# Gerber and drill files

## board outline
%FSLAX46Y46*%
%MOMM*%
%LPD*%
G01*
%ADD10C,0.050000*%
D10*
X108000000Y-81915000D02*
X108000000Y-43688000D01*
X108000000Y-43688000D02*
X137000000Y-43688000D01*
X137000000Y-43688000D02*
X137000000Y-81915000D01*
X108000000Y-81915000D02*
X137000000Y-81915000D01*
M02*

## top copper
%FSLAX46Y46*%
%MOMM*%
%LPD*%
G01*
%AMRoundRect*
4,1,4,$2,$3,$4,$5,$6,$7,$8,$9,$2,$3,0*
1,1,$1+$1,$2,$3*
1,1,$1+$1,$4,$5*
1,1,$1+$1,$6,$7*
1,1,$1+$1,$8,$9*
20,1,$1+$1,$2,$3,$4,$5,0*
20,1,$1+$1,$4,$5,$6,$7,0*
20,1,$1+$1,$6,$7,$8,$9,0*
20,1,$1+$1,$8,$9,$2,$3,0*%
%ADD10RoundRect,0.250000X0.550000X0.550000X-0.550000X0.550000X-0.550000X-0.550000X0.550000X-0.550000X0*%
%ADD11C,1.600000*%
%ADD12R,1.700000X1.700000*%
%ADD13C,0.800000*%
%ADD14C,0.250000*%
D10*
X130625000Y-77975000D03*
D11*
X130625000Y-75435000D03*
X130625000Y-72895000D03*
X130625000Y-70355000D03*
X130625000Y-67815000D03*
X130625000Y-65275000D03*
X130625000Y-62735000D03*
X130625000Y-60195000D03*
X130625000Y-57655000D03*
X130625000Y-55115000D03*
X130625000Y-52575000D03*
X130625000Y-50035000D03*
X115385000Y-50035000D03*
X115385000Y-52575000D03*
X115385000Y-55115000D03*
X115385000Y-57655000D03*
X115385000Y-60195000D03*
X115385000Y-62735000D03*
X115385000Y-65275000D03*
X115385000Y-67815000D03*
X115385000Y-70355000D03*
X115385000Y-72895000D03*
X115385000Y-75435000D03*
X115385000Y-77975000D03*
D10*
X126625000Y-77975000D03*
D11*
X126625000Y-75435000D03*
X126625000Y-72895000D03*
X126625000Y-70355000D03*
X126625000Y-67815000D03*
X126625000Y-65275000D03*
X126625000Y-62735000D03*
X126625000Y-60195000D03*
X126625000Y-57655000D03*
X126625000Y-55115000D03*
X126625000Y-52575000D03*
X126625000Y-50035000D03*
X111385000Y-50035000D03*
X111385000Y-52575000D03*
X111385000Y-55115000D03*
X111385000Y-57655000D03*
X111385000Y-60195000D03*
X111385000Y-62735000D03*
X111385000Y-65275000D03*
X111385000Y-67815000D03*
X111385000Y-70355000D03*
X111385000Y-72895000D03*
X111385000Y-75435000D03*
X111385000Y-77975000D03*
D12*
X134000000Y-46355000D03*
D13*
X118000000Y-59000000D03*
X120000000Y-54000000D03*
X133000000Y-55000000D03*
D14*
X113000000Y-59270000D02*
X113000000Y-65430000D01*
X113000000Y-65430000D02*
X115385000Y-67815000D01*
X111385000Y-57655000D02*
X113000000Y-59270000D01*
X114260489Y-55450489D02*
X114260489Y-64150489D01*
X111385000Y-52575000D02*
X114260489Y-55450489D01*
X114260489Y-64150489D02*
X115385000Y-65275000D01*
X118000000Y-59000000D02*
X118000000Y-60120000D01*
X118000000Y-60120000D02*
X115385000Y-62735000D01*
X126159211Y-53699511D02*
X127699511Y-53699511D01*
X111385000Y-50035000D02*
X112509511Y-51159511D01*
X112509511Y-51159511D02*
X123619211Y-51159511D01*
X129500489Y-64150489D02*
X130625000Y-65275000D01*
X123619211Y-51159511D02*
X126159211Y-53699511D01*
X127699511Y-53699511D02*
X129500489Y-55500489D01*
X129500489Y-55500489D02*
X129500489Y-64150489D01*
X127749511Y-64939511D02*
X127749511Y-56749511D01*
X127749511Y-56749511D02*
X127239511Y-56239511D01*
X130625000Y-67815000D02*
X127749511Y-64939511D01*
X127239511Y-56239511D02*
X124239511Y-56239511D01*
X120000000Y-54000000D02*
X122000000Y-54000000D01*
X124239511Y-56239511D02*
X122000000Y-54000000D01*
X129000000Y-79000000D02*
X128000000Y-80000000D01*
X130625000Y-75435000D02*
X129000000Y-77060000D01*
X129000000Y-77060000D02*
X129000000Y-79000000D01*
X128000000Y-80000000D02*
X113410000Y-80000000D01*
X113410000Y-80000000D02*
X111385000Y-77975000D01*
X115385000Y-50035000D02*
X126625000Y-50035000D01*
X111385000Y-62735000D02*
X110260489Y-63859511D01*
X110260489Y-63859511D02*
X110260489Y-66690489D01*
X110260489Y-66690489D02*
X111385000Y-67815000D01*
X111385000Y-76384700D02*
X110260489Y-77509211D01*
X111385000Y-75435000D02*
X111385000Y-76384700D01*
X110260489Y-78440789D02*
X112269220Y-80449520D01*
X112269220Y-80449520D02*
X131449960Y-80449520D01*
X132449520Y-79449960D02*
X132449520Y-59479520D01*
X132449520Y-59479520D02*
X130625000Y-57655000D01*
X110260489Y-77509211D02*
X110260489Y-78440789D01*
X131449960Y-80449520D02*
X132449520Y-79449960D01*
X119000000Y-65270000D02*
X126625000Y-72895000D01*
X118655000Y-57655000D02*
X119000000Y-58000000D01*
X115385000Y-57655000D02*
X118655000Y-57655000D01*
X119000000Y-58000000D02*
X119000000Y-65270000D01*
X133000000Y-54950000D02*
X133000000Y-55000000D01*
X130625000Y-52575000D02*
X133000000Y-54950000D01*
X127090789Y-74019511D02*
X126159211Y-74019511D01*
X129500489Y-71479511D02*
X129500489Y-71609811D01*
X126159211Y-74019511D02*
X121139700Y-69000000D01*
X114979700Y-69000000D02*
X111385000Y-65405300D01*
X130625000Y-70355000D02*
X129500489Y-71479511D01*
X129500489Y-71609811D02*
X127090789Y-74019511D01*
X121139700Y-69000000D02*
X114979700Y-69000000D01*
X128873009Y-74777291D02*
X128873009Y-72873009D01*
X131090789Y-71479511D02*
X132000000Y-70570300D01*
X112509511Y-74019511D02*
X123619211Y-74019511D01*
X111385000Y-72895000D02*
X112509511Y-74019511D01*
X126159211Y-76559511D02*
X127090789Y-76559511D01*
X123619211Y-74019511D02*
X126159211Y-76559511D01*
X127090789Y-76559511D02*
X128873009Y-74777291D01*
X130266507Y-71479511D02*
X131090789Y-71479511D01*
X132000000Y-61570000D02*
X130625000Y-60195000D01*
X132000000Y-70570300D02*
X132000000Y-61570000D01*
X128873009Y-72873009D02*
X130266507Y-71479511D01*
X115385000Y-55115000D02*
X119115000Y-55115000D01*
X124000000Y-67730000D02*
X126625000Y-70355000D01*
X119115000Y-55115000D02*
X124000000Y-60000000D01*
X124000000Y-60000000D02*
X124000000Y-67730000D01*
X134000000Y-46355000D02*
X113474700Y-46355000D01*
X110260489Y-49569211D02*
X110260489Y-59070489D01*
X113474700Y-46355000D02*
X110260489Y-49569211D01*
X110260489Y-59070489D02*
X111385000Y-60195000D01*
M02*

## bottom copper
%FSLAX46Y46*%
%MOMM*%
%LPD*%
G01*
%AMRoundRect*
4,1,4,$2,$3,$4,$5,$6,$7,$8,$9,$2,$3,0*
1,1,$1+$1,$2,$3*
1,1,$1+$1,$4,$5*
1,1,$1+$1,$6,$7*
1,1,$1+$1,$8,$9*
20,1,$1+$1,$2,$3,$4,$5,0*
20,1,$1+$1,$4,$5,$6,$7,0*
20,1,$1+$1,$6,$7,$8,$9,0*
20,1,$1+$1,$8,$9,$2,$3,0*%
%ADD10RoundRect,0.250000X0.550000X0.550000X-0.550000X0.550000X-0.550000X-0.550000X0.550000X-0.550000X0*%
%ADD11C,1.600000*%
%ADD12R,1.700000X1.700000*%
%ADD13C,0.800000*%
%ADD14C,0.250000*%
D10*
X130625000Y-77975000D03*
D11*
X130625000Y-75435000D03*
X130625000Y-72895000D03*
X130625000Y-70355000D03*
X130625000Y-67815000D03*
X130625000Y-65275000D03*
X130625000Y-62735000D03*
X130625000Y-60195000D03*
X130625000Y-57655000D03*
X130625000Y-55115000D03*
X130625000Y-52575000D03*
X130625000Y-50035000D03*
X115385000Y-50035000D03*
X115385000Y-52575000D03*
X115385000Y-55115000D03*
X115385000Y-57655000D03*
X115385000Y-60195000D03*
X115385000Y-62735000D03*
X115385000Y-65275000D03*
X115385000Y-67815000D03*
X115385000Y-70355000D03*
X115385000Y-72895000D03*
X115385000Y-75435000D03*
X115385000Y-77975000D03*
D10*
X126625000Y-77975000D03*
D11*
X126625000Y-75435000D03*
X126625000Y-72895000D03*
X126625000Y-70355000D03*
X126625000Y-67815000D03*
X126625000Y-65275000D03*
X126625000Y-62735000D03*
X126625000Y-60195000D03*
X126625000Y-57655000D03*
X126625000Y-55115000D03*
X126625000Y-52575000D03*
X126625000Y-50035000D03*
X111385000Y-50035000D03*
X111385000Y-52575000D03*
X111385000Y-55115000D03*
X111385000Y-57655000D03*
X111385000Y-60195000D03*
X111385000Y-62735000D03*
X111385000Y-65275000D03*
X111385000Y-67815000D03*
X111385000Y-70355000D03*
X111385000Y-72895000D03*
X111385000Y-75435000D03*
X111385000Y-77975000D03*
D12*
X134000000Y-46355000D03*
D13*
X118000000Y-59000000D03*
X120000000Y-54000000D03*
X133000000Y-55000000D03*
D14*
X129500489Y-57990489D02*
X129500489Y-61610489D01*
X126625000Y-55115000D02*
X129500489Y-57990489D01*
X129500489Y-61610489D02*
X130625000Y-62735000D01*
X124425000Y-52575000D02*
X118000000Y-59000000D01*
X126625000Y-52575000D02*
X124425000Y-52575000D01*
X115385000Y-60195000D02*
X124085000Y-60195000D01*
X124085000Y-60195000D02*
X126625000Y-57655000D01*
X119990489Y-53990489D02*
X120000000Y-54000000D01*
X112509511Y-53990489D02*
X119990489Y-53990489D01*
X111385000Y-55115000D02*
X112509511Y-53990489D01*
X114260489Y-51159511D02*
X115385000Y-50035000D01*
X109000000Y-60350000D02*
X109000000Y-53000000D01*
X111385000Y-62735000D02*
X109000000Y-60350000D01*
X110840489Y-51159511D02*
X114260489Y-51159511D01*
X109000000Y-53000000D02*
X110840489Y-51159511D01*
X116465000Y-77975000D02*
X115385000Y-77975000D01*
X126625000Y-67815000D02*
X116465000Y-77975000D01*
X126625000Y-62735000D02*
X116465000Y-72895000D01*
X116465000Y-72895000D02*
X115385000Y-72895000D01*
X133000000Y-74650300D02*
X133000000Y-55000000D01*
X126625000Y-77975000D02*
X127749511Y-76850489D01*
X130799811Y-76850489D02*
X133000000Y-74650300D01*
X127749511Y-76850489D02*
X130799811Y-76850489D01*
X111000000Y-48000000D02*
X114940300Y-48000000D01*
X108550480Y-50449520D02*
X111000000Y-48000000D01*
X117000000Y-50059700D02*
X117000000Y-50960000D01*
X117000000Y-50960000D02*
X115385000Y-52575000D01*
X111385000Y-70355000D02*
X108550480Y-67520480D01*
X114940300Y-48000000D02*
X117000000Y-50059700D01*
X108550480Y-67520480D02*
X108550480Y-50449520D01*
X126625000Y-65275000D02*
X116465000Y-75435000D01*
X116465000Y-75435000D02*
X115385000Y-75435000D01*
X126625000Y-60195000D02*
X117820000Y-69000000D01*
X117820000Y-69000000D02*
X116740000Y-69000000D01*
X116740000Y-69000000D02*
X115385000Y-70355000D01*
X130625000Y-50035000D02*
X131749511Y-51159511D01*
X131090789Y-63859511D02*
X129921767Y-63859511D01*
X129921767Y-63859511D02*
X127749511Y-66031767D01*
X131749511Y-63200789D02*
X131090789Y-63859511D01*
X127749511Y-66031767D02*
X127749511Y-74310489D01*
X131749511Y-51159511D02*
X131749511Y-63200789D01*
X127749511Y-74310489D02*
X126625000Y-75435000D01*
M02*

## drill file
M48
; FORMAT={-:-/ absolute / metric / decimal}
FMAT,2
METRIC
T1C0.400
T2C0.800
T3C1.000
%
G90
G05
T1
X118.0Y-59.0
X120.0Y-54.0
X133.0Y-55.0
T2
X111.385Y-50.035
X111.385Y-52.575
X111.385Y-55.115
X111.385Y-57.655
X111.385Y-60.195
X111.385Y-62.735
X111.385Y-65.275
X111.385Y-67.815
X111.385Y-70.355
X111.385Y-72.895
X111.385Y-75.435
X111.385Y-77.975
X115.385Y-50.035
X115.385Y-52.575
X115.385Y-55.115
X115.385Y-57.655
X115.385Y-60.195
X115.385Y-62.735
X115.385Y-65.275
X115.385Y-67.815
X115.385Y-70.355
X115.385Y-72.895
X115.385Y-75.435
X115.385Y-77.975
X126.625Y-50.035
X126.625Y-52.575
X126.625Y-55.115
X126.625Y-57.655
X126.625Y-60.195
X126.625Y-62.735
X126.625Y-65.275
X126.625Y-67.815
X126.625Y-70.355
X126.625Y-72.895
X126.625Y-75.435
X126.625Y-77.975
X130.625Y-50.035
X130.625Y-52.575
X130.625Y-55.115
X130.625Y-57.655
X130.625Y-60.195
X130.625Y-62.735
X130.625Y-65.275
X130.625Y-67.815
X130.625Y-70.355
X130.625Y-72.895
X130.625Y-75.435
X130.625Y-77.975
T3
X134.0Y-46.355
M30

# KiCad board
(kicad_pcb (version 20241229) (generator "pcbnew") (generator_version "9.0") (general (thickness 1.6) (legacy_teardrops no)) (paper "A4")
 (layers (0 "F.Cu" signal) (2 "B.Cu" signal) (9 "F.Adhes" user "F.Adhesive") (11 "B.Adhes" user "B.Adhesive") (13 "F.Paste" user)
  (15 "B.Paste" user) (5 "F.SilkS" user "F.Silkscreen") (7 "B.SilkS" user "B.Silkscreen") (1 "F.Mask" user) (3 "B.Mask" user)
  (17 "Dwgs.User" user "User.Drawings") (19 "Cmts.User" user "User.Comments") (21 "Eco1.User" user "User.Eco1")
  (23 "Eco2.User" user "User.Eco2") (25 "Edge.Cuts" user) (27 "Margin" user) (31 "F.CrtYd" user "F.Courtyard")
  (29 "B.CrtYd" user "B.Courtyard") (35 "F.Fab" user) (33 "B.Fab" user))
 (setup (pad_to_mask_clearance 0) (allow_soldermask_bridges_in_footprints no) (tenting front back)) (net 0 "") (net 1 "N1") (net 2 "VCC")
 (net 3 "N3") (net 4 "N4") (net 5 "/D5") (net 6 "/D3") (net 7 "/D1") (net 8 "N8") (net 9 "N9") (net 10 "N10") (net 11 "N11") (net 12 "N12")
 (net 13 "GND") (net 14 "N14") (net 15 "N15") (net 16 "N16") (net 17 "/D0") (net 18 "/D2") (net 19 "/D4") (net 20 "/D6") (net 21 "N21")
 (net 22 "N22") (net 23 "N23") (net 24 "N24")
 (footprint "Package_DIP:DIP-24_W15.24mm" (layer "F.Cu") (at 130.625 77.975 180)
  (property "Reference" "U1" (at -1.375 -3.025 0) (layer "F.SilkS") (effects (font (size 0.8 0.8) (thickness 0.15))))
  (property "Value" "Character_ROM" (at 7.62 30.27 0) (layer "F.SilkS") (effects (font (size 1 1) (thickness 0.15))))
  (pad "1" thru_hole roundrect (at 0 0 180) (size 1.6 1.6) (drill 0.8) (layers "*.Cu" "*.Mask") (remove_unused_layers no)
   (roundrect_rratio 0.15625) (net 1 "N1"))
  (pad "2" thru_hole circle (at 0 2.54 180) (size 1.6 1.6) (drill 0.8) (layers "*.Cu" "*.Mask") (remove_unused_layers no) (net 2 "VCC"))
  (pad "3" thru_hole circle (at 0 5.08 180) (size 1.6 1.6) (drill 0.8) (layers "*.Cu" "*.Mask") (remove_unused_layers no) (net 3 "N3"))
  (pad "4" thru_hole circle (at 0 7.62 180) (size 1.6 1.6) (drill 0.8) (layers "*.Cu" "*.Mask") (remove_unused_layers no) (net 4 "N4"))
  (pad "5" thru_hole circle (at 0 10.16 180) (size 1.6 1.6) (drill 0.8) (layers "*.Cu" "*.Mask") (remove_unused_layers no) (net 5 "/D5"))
  (pad "6" thru_hole circle (at 0 12.7 180) (size 1.6 1.6) (drill 0.8) (layers "*.Cu" "*.Mask") (remove_unused_layers no) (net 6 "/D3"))
  (pad "7" thru_hole circle (at 0 15.24 180) (size 1.6 1.6) (drill 0.8) (layers "*.Cu" "*.Mask") (remove_unused_layers no) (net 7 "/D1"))
  (pad "8" thru_hole circle (at 0 17.78 180) (size 1.6 1.6) (drill 0.8) (layers "*.Cu" "*.Mask") (remove_unused_layers no) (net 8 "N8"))
  (pad "9" thru_hole circle (at 0 20.32 180) (size 1.6 1.6) (drill 0.8) (layers "*.Cu" "*.Mask") (remove_unused_layers no) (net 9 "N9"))
  (pad "10" thru_hole circle (at 0 22.86 180) (size 1.6 1.6) (drill 0.8) (layers "*.Cu" "*.Mask") (remove_unused_layers no) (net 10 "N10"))
  (pad "11" thru_hole circle (at 0 25.4 180) (size 1.6 1.6) (drill 0.8) (layers "*.Cu" "*.Mask") (remove_unused_layers no) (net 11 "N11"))
  (pad "12" thru_hole circle (at 0 27.94 180) (size 1.6 1.6) (drill 0.8) (layers "*.Cu" "*.Mask") (remove_unused_layers no) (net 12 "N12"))
  (pad "13" thru_hole circle (at 15.24 27.94 180) (size 1.6 1.6) (drill 0.8) (layers "*.Cu" "*.Mask") (remove_unused_layers no)
   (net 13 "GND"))
  (pad "14" thru_hole circle (at 15.24 25.4 180) (size 1.6 1.6) (drill 0.8) (layers "*.Cu" "*.Mask") (remove_unused_layers no)
   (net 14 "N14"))
  (pad "15" thru_hole circle (at 15.24 22.86 180) (size 1.6 1.6) (drill 0.8) (layers "*.Cu" "*.Mask") (remove_unused_layers no)
   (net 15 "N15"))
  (pad "16" thru_hole circle (at 15.24 20.32 180) (size 1.6 1.6) (drill 0.8) (layers "*.Cu" "*.Mask") (remove_unused_layers no)
   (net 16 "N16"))
  (pad "17" thru_hole circle (at 15.24 17.78 180) (size 1.6 1.6) (drill 0.8) (layers "*.Cu" "*.Mask") (remove_unused_layers no)
   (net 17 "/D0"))
  (pad "18" thru_hole circle (at 15.24 15.24 180) (size 1.6 1.6) (drill 0.8) (layers "*.Cu" "*.Mask") (remove_unused_layers no)
   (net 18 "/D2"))
  (pad "19" thru_hole circle (at 15.24 12.7 180) (size 1.6 1.6) (drill 0.8) (layers "*.Cu" "*.Mask") (remove_unused_layers no)
   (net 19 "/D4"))
  (pad "20" thru_hole circle (at 15.24 10.16 180) (size 1.6 1.6) (drill 0.8) (layers "*.Cu" "*.Mask") (remove_unused_layers no)
   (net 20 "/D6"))
  (pad "21" thru_hole circle (at 15.24 7.62 180) (size 1.6 1.6) (drill 0.8) (layers "*.Cu" "*.Mask") (remove_unused_layers no)
   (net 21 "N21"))
  (pad "22" thru_hole circle (at 15.24 5.08 180) (size 1.6 1.6) (drill 0.8) (layers "*.Cu" "*.Mask") (remove_unused_layers no)
   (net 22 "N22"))
  (pad "23" thru_hole circle (at 15.24 2.54 180) (size 1.6 1.6) (drill 0.8) (layers "*.Cu" "*.Mask") (remove_unused_layers no)
   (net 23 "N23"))
  (pad "24" thru_hole circle (at 15.24 0 180) (size 1.6 1.6) (drill 0.8) (layers "*.Cu" "*.Mask") (remove_unused_layers no) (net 22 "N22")))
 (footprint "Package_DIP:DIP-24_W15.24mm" (layer "F.Cu") (at 126.625 77.975 180)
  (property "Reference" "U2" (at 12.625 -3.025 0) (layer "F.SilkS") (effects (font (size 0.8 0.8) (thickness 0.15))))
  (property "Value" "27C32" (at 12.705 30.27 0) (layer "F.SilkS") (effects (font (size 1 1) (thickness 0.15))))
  (pad "1" thru_hole roundrect (at 0 0 180) (size 1.6 1.6) (drill 0.8) (layers "*.Cu" "*.Mask") (remove_unused_layers no)
   (roundrect_rratio 0.15625) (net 11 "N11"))
  (pad "2" thru_hole circle (at 0 2.54 180) (size 1.6 1.6) (drill 0.8) (layers "*.Cu" "*.Mask") (remove_unused_layers no) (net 12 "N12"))
  (pad "3" thru_hole circle (at 0 5.08 180) (size 1.6 1.6) (drill 0.8) (layers "*.Cu" "*.Mask") (remove_unused_layers no) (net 16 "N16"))
  (pad "4" thru_hole circle (at 0 7.62 180) (size 1.6 1.6) (drill 0.8) (layers "*.Cu" "*.Mask") (remove_unused_layers no) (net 15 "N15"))
  (pad "5" thru_hole circle (at 0 10.16 180) (size 1.6 1.6) (drill 0.8) (layers "*.Cu" "*.Mask") (remove_unused_layers no) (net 22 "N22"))
  (pad "6" thru_hole circle (at 0 12.7 180) (size 1.6 1.6) (drill 0.8) (layers "*.Cu" "*.Mask") (remove_unused_layers no) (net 23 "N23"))
  (pad "7" thru_hole circle (at 0 15.24 180) (size 1.6 1.6) (drill 0.8) (layers "*.Cu" "*.Mask") (remove_unused_layers no) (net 22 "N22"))
  (pad "8" thru_hole circle (at 0 17.78 180) (size 1.6 1.6) (drill 0.8) (layers "*.Cu" "*.Mask") (remove_unused_layers no) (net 21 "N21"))
  (pad "9" thru_hole circle (at 0 20.32 180) (size 1.6 1.6) (drill 0.8) (layers "*.Cu" "*.Mask") (remove_unused_layers no) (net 17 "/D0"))
  (pad "10" thru_hole circle (at 0 22.86 180) (size 1.6 1.6) (drill 0.8) (layers "*.Cu" "*.Mask") (remove_unused_layers no) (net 7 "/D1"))
  (pad "11" thru_hole circle (at 0 25.4 180) (size 1.6 1.6) (drill 0.8) (layers "*.Cu" "*.Mask") (remove_unused_layers no) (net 18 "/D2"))
  (pad "12" thru_hole circle (at 0 27.94 180) (size 1.6 1.6) (drill 0.8) (layers "*.Cu" "*.Mask") (remove_unused_layers no) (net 13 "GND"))
  (pad "13" thru_hole circle (at 15.24 27.94 180) (size 1.6 1.6) (drill 0.8) (layers "*.Cu" "*.Mask") (remove_unused_layers no)
   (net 6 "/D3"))
  (pad "14" thru_hole circle (at 15.24 25.4 180) (size 1.6 1.6) (drill 0.8) (layers "*.Cu" "*.Mask") (remove_unused_layers no)
   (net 19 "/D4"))
  (pad "15" thru_hole circle (at 15.24 22.86 180) (size 1.6 1.6) (drill 0.8) (layers "*.Cu" "*.Mask") (remove_unused_layers no)
   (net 5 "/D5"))
  (pad "16" thru_hole circle (at 15.24 20.32 180) (size 1.6 1.6) (drill 0.8) (layers "*.Cu" "*.Mask") (remove_unused_layers no)
   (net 20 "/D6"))
  (pad "17" thru_hole circle (at 15.24 17.78 180) (size 1.6 1.6) (drill 0.8) (layers "*.Cu" "*.Mask") (remove_unused_layers no)
   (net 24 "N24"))
  (pad "18" thru_hole circle (at 15.24 15.24 180) (size 1.6 1.6) (drill 0.8) (layers "*.Cu" "*.Mask") (remove_unused_layers no)
   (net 13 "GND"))
  (pad "19" thru_hole circle (at 15.24 12.7 180) (size 1.6 1.6) (drill 0.8) (layers "*.Cu" "*.Mask") (remove_unused_layers no) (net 4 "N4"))
  (pad "20" thru_hole circle (at 15.24 10.16 180) (size 1.6 1.6) (drill 0.8) (layers "*.Cu" "*.Mask") (remove_unused_layers no)
   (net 13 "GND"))
  (pad "21" thru_hole circle (at 15.24 7.62 180) (size 1.6 1.6) (drill 0.8) (layers "*.Cu" "*.Mask") (remove_unused_layers no)
   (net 14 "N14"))
  (pad "22" thru_hole circle (at 15.24 5.08 180) (size 1.6 1.6) (drill 0.8) (layers "*.Cu" "*.Mask") (remove_unused_layers no) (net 8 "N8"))
  (pad "23" thru_hole circle (at 15.24 2.54 180) (size 1.6 1.6) (drill 0.8) (layers "*.Cu" "*.Mask") (remove_unused_layers no) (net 9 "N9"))
  (pad "24" thru_hole circle (at 15.24 0 180) (size 1.6 1.6) (drill 0.8) (layers "*.Cu" "*.Mask") (remove_unused_layers no) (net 2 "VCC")))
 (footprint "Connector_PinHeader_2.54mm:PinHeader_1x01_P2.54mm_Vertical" (layer "F.Cu") (at 134 46.355)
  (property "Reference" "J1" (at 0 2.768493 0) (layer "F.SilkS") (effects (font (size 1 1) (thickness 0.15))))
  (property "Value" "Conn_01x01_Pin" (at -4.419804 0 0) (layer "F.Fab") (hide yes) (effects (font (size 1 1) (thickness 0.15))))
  (pad "1" thru_hole rect (at 0 0) (size 1.7 1.7) (drill 1) (layers "*.Cu" "*.Mask") (remove_unused_layers no) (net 24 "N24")))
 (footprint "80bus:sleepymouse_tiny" (layer "F.Cu") (at 120.905854 71.728712)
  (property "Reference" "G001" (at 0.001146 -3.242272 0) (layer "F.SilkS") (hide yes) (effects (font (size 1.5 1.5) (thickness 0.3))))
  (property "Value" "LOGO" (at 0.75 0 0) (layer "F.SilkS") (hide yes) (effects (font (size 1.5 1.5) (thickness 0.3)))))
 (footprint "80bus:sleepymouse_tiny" (layer "F.Cu") (at 121.095634 56.101873)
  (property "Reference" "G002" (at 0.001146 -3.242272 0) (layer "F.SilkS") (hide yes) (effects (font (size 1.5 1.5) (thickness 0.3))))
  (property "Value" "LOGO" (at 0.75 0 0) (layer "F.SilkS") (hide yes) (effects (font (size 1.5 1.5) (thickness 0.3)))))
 (gr_line (start 108 81.915) (end 108 43.688) (stroke (width 0.05) (type solid)) (layer "Edge.Cuts"))
 (gr_line (start 108 43.688) (end 137 43.688) (stroke (width 0.05) (type solid)) (layer "Edge.Cuts"))
 (gr_line (start 137 43.688) (end 137 81.915) (stroke (width 0.05) (type solid)) (layer "Edge.Cuts"))
 (gr_line (start 108 81.915) (end 137 81.915) (stroke (width 0.05) (type solid)) (layer "Edge.Cuts"))
 (segment (start 113 59.27) (end 113 65.43) (width 0.25) (layer "F.Cu") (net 20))
 (segment (start 113 65.43) (end 115.385 67.815) (width 0.25) (layer "F.Cu") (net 20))
 (segment (start 111.385 57.655) (end 113 59.27) (width 0.25) (layer "F.Cu") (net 20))
 (segment (start 114.260489 55.450489) (end 114.260489 64.150489) (width 0.25) (layer "F.Cu") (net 19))
 (segment (start 111.385 52.575) (end 114.260489 55.450489) (width 0.25) (layer "F.Cu") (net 19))
 (segment (start 114.260489 64.150489) (end 115.385 65.275) (width 0.25) (layer "F.Cu") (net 19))
 (segment (start 129.500489 57.990489) (end 129.500489 61.610489) (width 0.25) (layer "B.Cu") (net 7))
 (segment (start 126.625 55.115) (end 129.500489 57.990489) (width 0.25) (layer "B.Cu") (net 7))
 (segment (start 129.500489 61.610489) (end 130.625 62.735) (width 0.25) (layer "B.Cu") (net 7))
 (segment (start 118 59) (end 118 60.12) (width 0.25) (layer "F.Cu") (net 18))
 (segment (start 118 60.12) (end 115.385 62.735) (width 0.25) (layer "F.Cu") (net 18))
 (via (at 118 59) (size 0.8) (drill 0.4) (layers "F.Cu" "B.Cu") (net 18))
 (segment (start 124.425 52.575) (end 118 59) (width 0.25) (layer "B.Cu") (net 18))
 (segment (start 126.625 52.575) (end 124.425 52.575) (width 0.25) (layer "B.Cu") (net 18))
 (segment (start 126.159211 53.699511) (end 127.699511 53.699511) (width 0.25) (layer "F.Cu") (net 6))
 (segment (start 111.385 50.035) (end 112.509511 51.159511) (width 0.25) (layer "F.Cu") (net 6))
 (segment (start 112.509511 51.159511) (end 123.619211 51.159511) (width 0.25) (layer "F.Cu") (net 6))
 (segment (start 129.500489 64.150489) (end 130.625 65.275) (width 0.25) (layer "F.Cu") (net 6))
 (segment (start 123.619211 51.159511) (end 126.159211 53.699511) (width 0.25) (layer "F.Cu") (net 6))
 (segment (start 127.699511 53.699511) (end 129.500489 55.500489) (width 0.25) (layer "F.Cu") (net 6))
 (segment (start 129.500489 55.500489) (end 129.500489 64.150489) (width 0.25) (layer "F.Cu") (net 6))
 (segment (start 115.385 60.195) (end 124.085 60.195) (width 0.25) (layer "B.Cu") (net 17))
 (segment (start 124.085 60.195) (end 126.625 57.655) (width 0.25) (layer "B.Cu") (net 17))
 (segment (start 127.749511 64.939511) (end 127.749511 56.749511) (width 0.25) (layer "F.Cu") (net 5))
 (segment (start 127.749511 56.749511) (end 127.239511 56.239511) (width 0.25) (layer "F.Cu") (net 5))
 (segment (start 130.625 67.815) (end 127.749511 64.939511) (width 0.25) (layer "F.Cu") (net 5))
 (segment (start 127.239511 56.239511) (end 124.239511 56.239511) (width 0.25) (layer "F.Cu") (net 5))
 (segment (start 120 54) (end 122 54) (width 0.25) (layer "F.Cu") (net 5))
 (segment (start 124.239511 56.239511) (end 122 54) (width 0.25) (layer "F.Cu") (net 5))
 (via (at 120 54) (size 0.8) (drill 0.4) (layers "F.Cu" "B.Cu") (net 5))
 (segment (start 119.990489 53.990489) (end 120 54) (width 0.25) (layer "B.Cu") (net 5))
 (segment (start 112.509511 53.990489) (end 119.990489 53.990489) (width 0.25) (layer "B.Cu") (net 5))
 (segment (start 111.385 55.115) (end 112.509511 53.990489) (width 0.25) (layer "B.Cu") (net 5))
 (segment (start 129 79) (end 128 80) (width 0.25) (layer "F.Cu") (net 2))
 (segment (start 130.625 75.435) (end 129 77.06) (width 0.25) (layer "F.Cu") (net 2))
 (segment (start 129 77.06) (end 129 79) (width 0.25) (layer "F.Cu") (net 2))
 (segment (start 128 80) (end 113.41 80) (width 0.25) (layer "F.Cu") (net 2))
 (segment (start 113.41 80) (end 111.385 77.975) (width 0.25) (layer "F.Cu") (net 2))
 (segment (start 115.385 50.035) (end 126.625 50.035) (width 0.25) (layer "F.Cu") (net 13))
 (segment (start 111.385 62.735) (end 110.260489 63.859511) (width 0.25) (layer "F.Cu") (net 13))
 (segment (start 110.260489 63.859511) (end 110.260489 66.690489) (width 0.25) (layer "F.Cu") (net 13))
 (segment (start 110.260489 66.690489) (end 111.385 67.815) (width 0.25) (layer "F.Cu") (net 13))
 (segment (start 114.260489 51.159511) (end 115.385 50.035) (width 0.25) (layer "B.Cu") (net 13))
 (segment (start 109 60.35) (end 109 53) (width 0.25) (layer "B.Cu") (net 13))
 (segment (start 111.385 62.735) (end 109 60.35) (width 0.25) (layer "B.Cu") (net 13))
 (segment (start 110.840489 51.159511) (end 114.260489 51.159511) (width 0.25) (layer "B.Cu") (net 13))
 (segment (start 109 53) (end 110.840489 51.159511) (width 0.25) (layer "B.Cu") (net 13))
 (segment (start 116.465 77.975) (end 115.385 77.975) (width 0.25) (layer "B.Cu") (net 22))
 (segment (start 126.625 67.815) (end 116.465 77.975) (width 0.25) (layer "B.Cu") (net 22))
 (segment (start 126.625 62.735) (end 116.465 72.895) (width 0.25) (layer "B.Cu") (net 22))
 (segment (start 116.465 72.895) (end 115.385 72.895) (width 0.25) (layer "B.Cu") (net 22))
 (segment (start 111.385 76.3847) (end 110.260489 77.509211) (width 0.25) (layer "F.Cu") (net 9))
 (segment (start 111.385 75.435) (end 111.385 76.3847) (width 0.25) (layer "F.Cu") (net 9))
 (segment (start 110.260489 78.440789) (end 112.26922 80.44952) (width 0.25) (layer "F.Cu") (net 9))
 (segment (start 112.26922 80.44952) (end 131.44996 80.44952) (width 0.25) (layer "F.Cu") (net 9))
 (segment (start 132.44952 79.44996) (end 132.44952 59.47952) (width 0.25) (layer "F.Cu") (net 9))
 (segment (start 132.44952 59.47952) (end 130.625 57.655) (width 0.25) (layer "F.Cu") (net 9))
 (segment (start 110.260489 77.509211) (end 110.260489 78.440789) (width 0.25) (layer "F.Cu") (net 9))
 (segment (start 131.44996 80.44952) (end 132.44952 79.44996) (width 0.25) (layer "F.Cu") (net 9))
 (segment (start 119 65.27) (end 126.625 72.895) (width 0.25) (layer "F.Cu") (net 16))
 (segment (start 118.655 57.655) (end 119 58) (width 0.25) (layer "F.Cu") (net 16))
 (segment (start 115.385 57.655) (end 118.655 57.655) (width 0.25) (layer "F.Cu") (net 16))
 (segment (start 119 58) (end 119 65.27) (width 0.25) (layer "F.Cu") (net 16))
 (segment (start 133 54.95) (end 133 55) (width 0.25) (layer "F.Cu") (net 11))
 (segment (start 130.625 52.575) (end 133 54.95) (width 0.25) (layer "F.Cu") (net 11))
 (via (at 133 55) (size 0.8) (drill 0.4) (layers "F.Cu" "B.Cu") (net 11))
 (segment (start 133 74.6503) (end 133 55) (width 0.25) (layer "B.Cu") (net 11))
 (segment (start 126.625 77.975) (end 127.749511 76.850489) (width 0.25) (layer "B.Cu") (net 11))
 (segment (start 130.799811 76.850489) (end 133 74.6503) (width 0.25) (layer "B.Cu") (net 11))
 (segment (start 127.749511 76.850489) (end 130.799811 76.850489) (width 0.25) (layer "B.Cu") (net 11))
 (segment (start 111 48) (end 114.9403 48) (width 0.25) (layer "B.Cu") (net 14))
 (segment (start 108.55048 50.44952) (end 111 48) (width 0.25) (layer "B.Cu") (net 14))
 (segment (start 117 50.0597) (end 117 50.96) (width 0.25) (layer "B.Cu") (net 14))
 (segment (start 117 50.96) (end 115.385 52.575) (width 0.25) (layer "B.Cu") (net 14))
 (segment (start 111.385 70.355) (end 108.55048 67.52048) (width 0.25) (layer "B.Cu") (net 14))
 (segment (start 114.9403 48) (end 117 50.0597) (width 0.25) (layer "B.Cu") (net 14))
 (segment (start 108.55048 67.52048) (end 108.55048 50.44952) (width 0.25) (layer "B.Cu") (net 14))
 (segment (start 126.625 65.275) (end 116.465 75.435) (width 0.25) (layer "B.Cu") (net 23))
 (segment (start 116.465 75.435) (end 115.385 75.435) (width 0.25) (layer "B.Cu") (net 23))
 (segment (start 126.625 60.195) (end 117.82 69) (width 0.25) (layer "B.Cu") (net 21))
 (segment (start 117.82 69) (end 116.74 69) (width 0.25) (layer "B.Cu") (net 21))
 (segment (start 116.74 69) (end 115.385 70.355) (width 0.25) (layer "B.Cu") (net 21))
 (segment (start 127.090789 74.019511) (end 126.159211 74.019511) (width 0.25) (layer "F.Cu") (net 4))
 (segment (start 129.500489 71.479511) (end 129.500489 71.609811) (width 0.25) (layer "F.Cu") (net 4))
 (segment (start 126.159211 74.019511) (end 121.1397 69) (width 0.25) (layer "F.Cu") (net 4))
 (segment (start 114.9797 69) (end 111.385 65.4053) (width 0.25) (layer "F.Cu") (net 4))
 (segment (start 130.625 70.355) (end 129.500489 71.479511) (width 0.25) (layer "F.Cu") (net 4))
 (segment (start 129.500489 71.609811) (end 127.090789 74.019511) (width 0.25) (layer "F.Cu") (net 4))
 (segment (start 121.1397 69) (end 114.9797 69) (width 0.25) (layer "F.Cu") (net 4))
 (segment (start 130.625 50.035) (end 131.749511 51.159511) (width 0.25) (layer "B.Cu") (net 12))
 (segment (start 131.090789 63.859511) (end 129.921767 63.859511) (width 0.25) (layer "B.Cu") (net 12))
 (segment (start 129.921767 63.859511) (end 127.749511 66.031767) (width 0.25) (layer "B.Cu") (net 12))
 (segment (start 131.749511 63.200789) (end 131.090789 63.859511) (width 0.25) (layer "B.Cu") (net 12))
 (segment (start 127.749511 66.031767) (end 127.749511 74.310489) (width 0.25) (layer "B.Cu") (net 12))
 (segment (start 131.749511 51.159511) (end 131.749511 63.200789) (width 0.25) (layer "B.Cu") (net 12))
 (segment (start 127.749511 74.310489) (end 126.625 75.435) (width 0.25) (layer "B.Cu") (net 12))
 (segment (start 128.873009 74.777291) (end 128.873009 72.873009) (width 0.25) (layer "F.Cu") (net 8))
 (segment (start 131.090789 71.479511) (end 132 70.5703) (width 0.25) (layer "F.Cu") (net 8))
 (segment (start 112.509511 74.019511) (end 123.619211 74.019511) (width 0.25) (layer "F.Cu") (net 8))
 (segment (start 111.385 72.895) (end 112.509511 74.019511) (width 0.25) (layer "F.Cu") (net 8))
 (segment (start 126.159211 76.559511) (end 127.090789 76.559511) (width 0.25) (layer "F.Cu") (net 8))
 (segment (start 123.619211 74.019511) (end 126.159211 76.559511) (width 0.25) (layer "F.Cu") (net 8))
 (segment (start 127.090789 76.559511) (end 128.873009 74.777291) (width 0.25) (layer "F.Cu") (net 8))
 (segment (start 130.266507 71.479511) (end 131.090789 71.479511) (width 0.25) (layer "F.Cu") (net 8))
 (segment (start 132 61.57) (end 130.625 60.195) (width 0.25) (layer "F.Cu") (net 8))
 (segment (start 132 70.5703) (end 132 61.57) (width 0.25) (layer "F.Cu") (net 8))
 (segment (start 128.873009 72.873009) (end 130.266507 71.479511) (width 0.25) (layer "F.Cu") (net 8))
 (segment (start 115.385 55.115) (end 119.115 55.115) (width 0.25) (layer "F.Cu") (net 15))
 (segment (start 124 67.73) (end 126.625 70.355) (width 0.25) (layer "F.Cu") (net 15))
 (segment (start 119.115 55.115) (end 124 60) (width 0.25) (layer "F.Cu") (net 15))
 (segment (start 124 60) (end 124 67.73) (width 0.25) (layer "F.Cu") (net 15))
 (segment (start 134 46.355) (end 113.4747 46.355) (width 0.25) (layer "F.Cu") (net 24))
 (segment (start 110.260489 49.569211) (end 110.260489 59.070489) (width 0.25) (layer "F.Cu") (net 24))
 (segment (start 113.4747 46.355) (end 110.260489 49.569211) (width 0.25) (layer "F.Cu") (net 24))
 (segment (start 110.260489 59.070489) (end 111.385 60.195) (width 0.25) (layer "F.Cu") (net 24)))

